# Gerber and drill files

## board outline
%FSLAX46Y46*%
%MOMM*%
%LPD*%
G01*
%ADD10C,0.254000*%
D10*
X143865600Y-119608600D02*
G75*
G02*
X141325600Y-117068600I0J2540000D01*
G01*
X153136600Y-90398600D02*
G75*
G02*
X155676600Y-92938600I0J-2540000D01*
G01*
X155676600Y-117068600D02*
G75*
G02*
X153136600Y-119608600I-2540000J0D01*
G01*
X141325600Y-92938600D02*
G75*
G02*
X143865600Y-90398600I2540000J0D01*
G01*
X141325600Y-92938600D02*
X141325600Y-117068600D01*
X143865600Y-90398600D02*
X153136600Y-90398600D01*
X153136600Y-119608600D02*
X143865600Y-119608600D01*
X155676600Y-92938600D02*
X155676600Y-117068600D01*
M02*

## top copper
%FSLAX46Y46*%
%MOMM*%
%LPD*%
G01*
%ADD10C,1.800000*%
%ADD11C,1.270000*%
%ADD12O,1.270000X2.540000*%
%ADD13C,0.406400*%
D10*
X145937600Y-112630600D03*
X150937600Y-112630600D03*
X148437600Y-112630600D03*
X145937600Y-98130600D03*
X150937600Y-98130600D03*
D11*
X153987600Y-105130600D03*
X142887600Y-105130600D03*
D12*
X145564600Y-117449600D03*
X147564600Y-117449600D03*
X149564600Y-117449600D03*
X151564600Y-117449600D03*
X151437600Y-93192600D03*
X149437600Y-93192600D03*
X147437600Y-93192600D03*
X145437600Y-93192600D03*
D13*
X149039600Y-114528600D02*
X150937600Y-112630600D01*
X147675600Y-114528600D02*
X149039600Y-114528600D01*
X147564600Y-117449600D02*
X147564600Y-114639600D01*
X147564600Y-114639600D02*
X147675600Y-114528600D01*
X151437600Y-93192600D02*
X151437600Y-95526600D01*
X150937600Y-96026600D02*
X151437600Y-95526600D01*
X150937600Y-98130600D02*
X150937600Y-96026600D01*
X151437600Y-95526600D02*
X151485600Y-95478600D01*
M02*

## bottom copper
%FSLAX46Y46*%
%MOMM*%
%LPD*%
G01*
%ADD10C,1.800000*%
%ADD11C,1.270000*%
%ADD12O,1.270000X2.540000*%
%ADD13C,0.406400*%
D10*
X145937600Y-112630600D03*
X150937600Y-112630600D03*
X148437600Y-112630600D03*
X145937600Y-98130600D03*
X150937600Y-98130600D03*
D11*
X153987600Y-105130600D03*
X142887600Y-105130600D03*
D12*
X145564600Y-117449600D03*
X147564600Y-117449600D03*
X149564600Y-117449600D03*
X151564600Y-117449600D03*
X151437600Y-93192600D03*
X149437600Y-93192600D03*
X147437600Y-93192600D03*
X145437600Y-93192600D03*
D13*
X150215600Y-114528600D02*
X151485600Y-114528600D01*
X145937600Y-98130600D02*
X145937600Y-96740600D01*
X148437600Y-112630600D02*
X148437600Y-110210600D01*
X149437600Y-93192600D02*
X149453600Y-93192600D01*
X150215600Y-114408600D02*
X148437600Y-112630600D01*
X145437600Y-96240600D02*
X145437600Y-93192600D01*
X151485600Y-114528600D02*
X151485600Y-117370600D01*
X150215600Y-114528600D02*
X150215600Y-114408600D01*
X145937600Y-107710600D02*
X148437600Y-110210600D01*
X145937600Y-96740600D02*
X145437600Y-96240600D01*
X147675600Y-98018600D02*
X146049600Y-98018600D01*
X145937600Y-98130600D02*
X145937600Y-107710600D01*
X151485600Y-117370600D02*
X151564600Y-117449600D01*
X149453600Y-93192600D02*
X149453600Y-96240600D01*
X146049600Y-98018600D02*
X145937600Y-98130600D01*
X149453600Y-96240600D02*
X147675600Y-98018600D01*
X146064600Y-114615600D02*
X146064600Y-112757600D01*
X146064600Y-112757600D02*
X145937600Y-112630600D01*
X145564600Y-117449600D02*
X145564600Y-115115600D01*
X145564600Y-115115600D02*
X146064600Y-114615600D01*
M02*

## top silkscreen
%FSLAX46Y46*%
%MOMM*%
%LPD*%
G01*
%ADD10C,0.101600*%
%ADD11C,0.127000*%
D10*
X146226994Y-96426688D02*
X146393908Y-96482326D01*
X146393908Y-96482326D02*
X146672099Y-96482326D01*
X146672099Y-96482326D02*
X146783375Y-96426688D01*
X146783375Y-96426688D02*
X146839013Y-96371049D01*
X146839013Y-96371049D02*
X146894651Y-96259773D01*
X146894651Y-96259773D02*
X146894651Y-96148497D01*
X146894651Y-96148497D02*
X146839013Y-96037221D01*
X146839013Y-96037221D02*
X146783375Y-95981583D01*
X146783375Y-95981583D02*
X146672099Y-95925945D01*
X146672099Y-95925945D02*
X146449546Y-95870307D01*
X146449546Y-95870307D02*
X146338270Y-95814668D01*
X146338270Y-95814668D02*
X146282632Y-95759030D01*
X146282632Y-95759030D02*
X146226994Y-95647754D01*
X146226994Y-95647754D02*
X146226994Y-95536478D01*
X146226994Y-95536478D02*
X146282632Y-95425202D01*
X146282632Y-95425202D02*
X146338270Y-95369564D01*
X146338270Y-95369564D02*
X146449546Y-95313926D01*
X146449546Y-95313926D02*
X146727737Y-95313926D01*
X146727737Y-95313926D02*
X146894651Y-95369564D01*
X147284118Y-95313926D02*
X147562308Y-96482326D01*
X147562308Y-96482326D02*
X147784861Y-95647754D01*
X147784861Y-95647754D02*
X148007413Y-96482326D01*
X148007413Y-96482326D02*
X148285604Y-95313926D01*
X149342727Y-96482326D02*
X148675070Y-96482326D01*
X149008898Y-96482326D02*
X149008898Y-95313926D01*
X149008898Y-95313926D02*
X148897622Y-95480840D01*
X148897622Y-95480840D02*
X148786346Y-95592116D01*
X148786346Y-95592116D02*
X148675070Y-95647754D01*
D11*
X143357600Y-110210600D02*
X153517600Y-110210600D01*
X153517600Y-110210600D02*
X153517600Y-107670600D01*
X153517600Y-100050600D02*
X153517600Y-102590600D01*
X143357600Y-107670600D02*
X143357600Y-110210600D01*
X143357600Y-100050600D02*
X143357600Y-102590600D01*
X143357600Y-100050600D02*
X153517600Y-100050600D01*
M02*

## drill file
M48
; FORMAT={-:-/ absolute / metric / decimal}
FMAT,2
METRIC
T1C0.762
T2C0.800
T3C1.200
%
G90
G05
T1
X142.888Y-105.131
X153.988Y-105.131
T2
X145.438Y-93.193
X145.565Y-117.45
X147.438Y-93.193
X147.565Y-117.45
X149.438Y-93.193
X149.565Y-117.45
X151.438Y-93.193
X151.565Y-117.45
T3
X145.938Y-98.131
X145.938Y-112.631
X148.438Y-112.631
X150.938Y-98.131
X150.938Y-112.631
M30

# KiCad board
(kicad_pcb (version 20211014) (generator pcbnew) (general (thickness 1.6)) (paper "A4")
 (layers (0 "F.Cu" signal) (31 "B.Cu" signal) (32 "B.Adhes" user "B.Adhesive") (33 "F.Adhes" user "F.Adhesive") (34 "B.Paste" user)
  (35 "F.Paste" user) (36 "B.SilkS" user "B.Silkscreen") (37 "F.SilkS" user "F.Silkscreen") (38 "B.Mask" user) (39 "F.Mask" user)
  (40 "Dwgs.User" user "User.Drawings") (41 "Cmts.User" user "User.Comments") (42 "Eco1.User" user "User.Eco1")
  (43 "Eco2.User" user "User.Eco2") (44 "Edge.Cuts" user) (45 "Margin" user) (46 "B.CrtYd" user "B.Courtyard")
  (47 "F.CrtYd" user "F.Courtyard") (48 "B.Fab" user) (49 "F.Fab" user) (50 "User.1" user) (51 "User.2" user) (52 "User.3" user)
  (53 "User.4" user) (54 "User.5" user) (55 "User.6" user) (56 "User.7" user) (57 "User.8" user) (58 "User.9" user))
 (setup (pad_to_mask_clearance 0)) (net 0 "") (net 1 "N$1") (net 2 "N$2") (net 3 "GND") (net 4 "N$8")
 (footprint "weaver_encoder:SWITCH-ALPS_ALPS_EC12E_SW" (layer "F.Cu") (at 148.4376 105.1306)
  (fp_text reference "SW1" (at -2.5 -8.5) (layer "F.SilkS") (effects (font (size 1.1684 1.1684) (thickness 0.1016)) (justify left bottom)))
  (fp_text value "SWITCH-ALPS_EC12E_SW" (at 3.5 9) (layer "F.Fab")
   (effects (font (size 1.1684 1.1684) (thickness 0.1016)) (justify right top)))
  (fp_line (start -5.08 5.08) (end 5.08 5.08) (layer "F.SilkS") (width 0.127))
  (fp_line (start 5.08 5.08) (end 5.08 2.54) (layer "F.SilkS") (width 0.127))
  (fp_line (start 5.08 -5.08) (end 5.08 -2.54) (layer "F.SilkS") (width 0.127))
  (fp_line (start -5.08 2.54) (end -5.08 5.08) (layer "F.SilkS") (width 0.127))
  (fp_line (start -5.08 -5.08) (end -5.08 -2.54) (layer "F.SilkS") (width 0.127))
  (fp_line (start -5.08 -5.08) (end 5.08 -5.08) (layer "F.SilkS") (width 0.127))
  (pad "A" thru_hole circle (at -2.5 7.5) (size 1.8 1.8) (drill 1.2) (layers *.Cu *.Mask) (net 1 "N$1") (solder_mask_margin 0.1016))
  (pad "B" thru_hole circle (at 2.5 7.5) (size 1.8 1.8) (drill 1.2) (layers *.Cu *.Mask) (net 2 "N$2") (solder_mask_margin 0.1016))
  (pad "C" thru_hole circle (at 0 7.5) (size 1.8 1.8) (drill 1.2) (layers *.Cu *.Mask) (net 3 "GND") (solder_mask_margin 0.1016))
  (pad "D" thru_hole circle (at -2.5 -7) (size 1.8 1.8) (drill 1.2) (layers *.Cu *.Mask) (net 3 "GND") (solder_mask_margin 0.1016))
  (pad "E" thru_hole circle (at 2.5 -7) (size 1.8 1.8) (drill 1.2) (layers *.Cu *.Mask) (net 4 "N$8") (solder_mask_margin 0.1016))
  (pad "GND1" thru_hole circle (at 5.55 0) (size 1.27 1.27) (drill 0.762) (layers *.Cu *.Mask) (solder_mask_margin 0.1016))
  (pad "GND2" thru_hole circle (at -5.55 0) (size 1.27 1.27) (drill 0.762) (layers *.Cu *.Mask) (solder_mask_margin 0.1016)))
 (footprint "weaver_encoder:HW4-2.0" (layer "B.Cu") (at 148.5646 117.4496)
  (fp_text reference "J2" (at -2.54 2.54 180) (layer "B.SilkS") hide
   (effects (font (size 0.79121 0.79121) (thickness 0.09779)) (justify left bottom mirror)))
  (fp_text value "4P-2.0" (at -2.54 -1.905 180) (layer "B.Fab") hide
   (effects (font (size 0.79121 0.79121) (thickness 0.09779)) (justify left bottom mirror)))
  (pad "1" thru_hole oval (at -3 0 270) (size 2.54 1.27) (drill 0.8) (layers *.Cu *.Mask) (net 1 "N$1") (solder_mask_margin 0.1016))
  (pad "2" thru_hole oval (at -1 0 270) (size 2.54 1.27) (drill 0.8) (layers *.Cu *.Mask) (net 2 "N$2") (solder_mask_margin 0.1016))
  (pad "3" thru_hole oval (at 1 0 270) (size 2.54 1.27) (drill 0.8) (layers *.Cu *.Mask) (solder_mask_margin 0.1016))
  (pad "4" thru_hole oval (at 3 0 270) (size 2.54 1.27) (drill 0.8) (layers *.Cu *.Mask) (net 3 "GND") (solder_mask_margin 0.1016)))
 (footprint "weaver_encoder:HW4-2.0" (layer "B.Cu") (at 148.4376 93.1926 180)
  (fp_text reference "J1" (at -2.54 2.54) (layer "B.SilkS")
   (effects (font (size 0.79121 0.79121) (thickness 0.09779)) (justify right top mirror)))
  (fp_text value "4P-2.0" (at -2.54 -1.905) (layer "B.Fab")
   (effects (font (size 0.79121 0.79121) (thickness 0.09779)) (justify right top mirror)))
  (pad "1" thru_hole oval (at -3 0 90) (size 2.54 1.27) (drill 0.8) (layers *.Cu *.Mask) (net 4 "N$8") (solder_mask_margin 0.1016))
  (pad "2" thru_hole oval (at -1 0 90) (size 2.54 1.27) (drill 0.8) (layers *.Cu *.Mask) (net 3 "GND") (solder_mask_margin 0.1016))
  (pad "3" thru_hole oval (at 1 0 90) (size 2.54 1.27) (drill 0.8) (layers *.Cu *.Mask) (solder_mask_margin 0.1016))
  (pad "4" thru_hole oval (at 3 0 90) (size 2.54 1.27) (drill 0.8) (layers *.Cu *.Mask) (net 3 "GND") (solder_mask_margin 0.1016)))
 (gr_arc (start 143.8656 119.6086) (mid 142.069549 118.864651) (end 141.3256 117.0686) (layer "Edge.Cuts") (width 0.254))
 (gr_arc (start 153.1366 90.3986) (mid 154.932651 91.142549) (end 155.6766 92.9386) (layer "Edge.Cuts") (width 0.254))
 (gr_arc (start 155.6766 117.0686) (mid 154.932651 118.864651) (end 153.1366 119.6086) (layer "Edge.Cuts") (width 0.254))
 (gr_arc (start 141.3256 92.9386) (mid 142.069549 91.142549) (end 143.8656 90.3986) (layer "Edge.Cuts") (width 0.254))
 (gr_line (start 141.3256 92.9386) (end 141.3256 117.0686) (layer "Edge.Cuts") (width 0.254))
 (gr_line (start 143.8656 90.3986) (end 153.1366 90.3986) (layer "Edge.Cuts") (width 0.254))
 (gr_line (start 153.1366 119.6086) (end 143.8656 119.6086) (layer "Edge.Cuts") (width 0.254))
 (gr_line (start 155.6766 92.9386) (end 155.6766 117.0686) (layer "Edge.Cuts") (width 0.254))
 (segment (start 150.2156 114.5286) (end 151.4856 114.5286) (width 0.4064) (layer "B.Cu") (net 3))
 (segment (start 145.9376 98.1306) (end 145.9376 96.7406) (width 0.4064) (layer "B.Cu") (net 3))
 (segment (start 148.4376 112.6306) (end 148.4376 110.2106) (width 0.4064) (layer "B.Cu") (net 3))
 (segment (start 149.4376 93.1926) (end 149.4536 93.1926) (width 0.4064) (layer "B.Cu") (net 3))
 (segment (start 150.2156 114.4086) (end 148.4376 112.6306) (width 0.4064) (layer "B.Cu") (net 3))
 (segment (start 145.4376 96.2406) (end 145.4376 93.1926) (width 0.4064) (layer "B.Cu") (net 3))
 (segment (start 151.4856 114.5286) (end 151.4856 117.3706) (width 0.4064) (layer "B.Cu") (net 3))
 (segment (start 150.2156 114.5286) (end 150.2156 114.4086) (width 0.4064) (layer "B.Cu") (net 3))
 (segment (start 145.9376 107.7106) (end 148.4376 110.2106) (width 0.4064) (layer "B.Cu") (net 3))
 (segment (start 145.9376 96.7406) (end 145.4376 96.2406) (width 0.4064) (layer "B.Cu") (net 3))
 (segment (start 147.6756 98.0186) (end 146.0496 98.0186) (width 0.4064) (layer "B.Cu") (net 3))
 (segment (start 145.9376 98.1306) (end 145.9376 107.7106) (width 0.4064) (layer "B.Cu") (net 3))
 (segment (start 151.4856 117.3706) (end 151.5646 117.4496) (width 0.4064) (layer "B.Cu") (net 3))
 (segment (start 149.4536 93.1926) (end 149.4536 96.2406) (width 0.4064) (layer "B.Cu") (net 3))
 (segment (start 146.0496 98.0186) (end 145.9376 98.1306) (width 0.4064) (layer "B.Cu") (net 3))
 (segment (start 149.4536 96.2406) (end 147.6756 98.0186) (width 0.4064) (layer "B.Cu") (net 3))
 (segment (start 149.0396 114.5286) (end 150.9376 112.6306) (width 0.4064) (layer "F.Cu") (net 2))
 (segment (start 147.6756 114.5286) (end 149.0396 114.5286) (width 0.4064) (layer "F.Cu") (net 2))
 (segment (start 147.5646 117.4496) (end 147.5646 114.6396) (width 0.4064) (layer "F.Cu") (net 2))
 (segment (start 147.5646 114.6396) (end 147.6756 114.5286) (width 0.4064) (layer "F.Cu") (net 2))
 (segment (start 146.0646 114.6156) (end 146.0646 112.7576) (width 0.4064) (layer "B.Cu") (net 1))
 (segment (start 146.0646 112.7576) (end 145.9376 112.6306) (width 0.4064) (layer "B.Cu") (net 1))
 (segment (start 145.5646 117.4496) (end 145.5646 115.1156) (width 0.4064) (layer "B.Cu") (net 1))
 (segment (start 145.5646 115.1156) (end 146.0646 114.6156) (width 0.4064) (layer "B.Cu") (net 1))
 (segment (start 151.4376 93.1926) (end 151.4376 95.5266) (width 0.4064) (layer "F.Cu") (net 4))
 (segment (start 150.9376 96.0266) (end 151.4376 95.5266) (width 0.4064) (layer "F.Cu") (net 4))
 (segment (start 150.9376 98.1306) (end 150.9376 96.0266) (width 0.4064) (layer "F.Cu") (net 4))
 (segment (start 151.4376 95.5266) (end 151.4856 95.4786) (width 0.4064) (layer "F.Cu") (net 4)))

